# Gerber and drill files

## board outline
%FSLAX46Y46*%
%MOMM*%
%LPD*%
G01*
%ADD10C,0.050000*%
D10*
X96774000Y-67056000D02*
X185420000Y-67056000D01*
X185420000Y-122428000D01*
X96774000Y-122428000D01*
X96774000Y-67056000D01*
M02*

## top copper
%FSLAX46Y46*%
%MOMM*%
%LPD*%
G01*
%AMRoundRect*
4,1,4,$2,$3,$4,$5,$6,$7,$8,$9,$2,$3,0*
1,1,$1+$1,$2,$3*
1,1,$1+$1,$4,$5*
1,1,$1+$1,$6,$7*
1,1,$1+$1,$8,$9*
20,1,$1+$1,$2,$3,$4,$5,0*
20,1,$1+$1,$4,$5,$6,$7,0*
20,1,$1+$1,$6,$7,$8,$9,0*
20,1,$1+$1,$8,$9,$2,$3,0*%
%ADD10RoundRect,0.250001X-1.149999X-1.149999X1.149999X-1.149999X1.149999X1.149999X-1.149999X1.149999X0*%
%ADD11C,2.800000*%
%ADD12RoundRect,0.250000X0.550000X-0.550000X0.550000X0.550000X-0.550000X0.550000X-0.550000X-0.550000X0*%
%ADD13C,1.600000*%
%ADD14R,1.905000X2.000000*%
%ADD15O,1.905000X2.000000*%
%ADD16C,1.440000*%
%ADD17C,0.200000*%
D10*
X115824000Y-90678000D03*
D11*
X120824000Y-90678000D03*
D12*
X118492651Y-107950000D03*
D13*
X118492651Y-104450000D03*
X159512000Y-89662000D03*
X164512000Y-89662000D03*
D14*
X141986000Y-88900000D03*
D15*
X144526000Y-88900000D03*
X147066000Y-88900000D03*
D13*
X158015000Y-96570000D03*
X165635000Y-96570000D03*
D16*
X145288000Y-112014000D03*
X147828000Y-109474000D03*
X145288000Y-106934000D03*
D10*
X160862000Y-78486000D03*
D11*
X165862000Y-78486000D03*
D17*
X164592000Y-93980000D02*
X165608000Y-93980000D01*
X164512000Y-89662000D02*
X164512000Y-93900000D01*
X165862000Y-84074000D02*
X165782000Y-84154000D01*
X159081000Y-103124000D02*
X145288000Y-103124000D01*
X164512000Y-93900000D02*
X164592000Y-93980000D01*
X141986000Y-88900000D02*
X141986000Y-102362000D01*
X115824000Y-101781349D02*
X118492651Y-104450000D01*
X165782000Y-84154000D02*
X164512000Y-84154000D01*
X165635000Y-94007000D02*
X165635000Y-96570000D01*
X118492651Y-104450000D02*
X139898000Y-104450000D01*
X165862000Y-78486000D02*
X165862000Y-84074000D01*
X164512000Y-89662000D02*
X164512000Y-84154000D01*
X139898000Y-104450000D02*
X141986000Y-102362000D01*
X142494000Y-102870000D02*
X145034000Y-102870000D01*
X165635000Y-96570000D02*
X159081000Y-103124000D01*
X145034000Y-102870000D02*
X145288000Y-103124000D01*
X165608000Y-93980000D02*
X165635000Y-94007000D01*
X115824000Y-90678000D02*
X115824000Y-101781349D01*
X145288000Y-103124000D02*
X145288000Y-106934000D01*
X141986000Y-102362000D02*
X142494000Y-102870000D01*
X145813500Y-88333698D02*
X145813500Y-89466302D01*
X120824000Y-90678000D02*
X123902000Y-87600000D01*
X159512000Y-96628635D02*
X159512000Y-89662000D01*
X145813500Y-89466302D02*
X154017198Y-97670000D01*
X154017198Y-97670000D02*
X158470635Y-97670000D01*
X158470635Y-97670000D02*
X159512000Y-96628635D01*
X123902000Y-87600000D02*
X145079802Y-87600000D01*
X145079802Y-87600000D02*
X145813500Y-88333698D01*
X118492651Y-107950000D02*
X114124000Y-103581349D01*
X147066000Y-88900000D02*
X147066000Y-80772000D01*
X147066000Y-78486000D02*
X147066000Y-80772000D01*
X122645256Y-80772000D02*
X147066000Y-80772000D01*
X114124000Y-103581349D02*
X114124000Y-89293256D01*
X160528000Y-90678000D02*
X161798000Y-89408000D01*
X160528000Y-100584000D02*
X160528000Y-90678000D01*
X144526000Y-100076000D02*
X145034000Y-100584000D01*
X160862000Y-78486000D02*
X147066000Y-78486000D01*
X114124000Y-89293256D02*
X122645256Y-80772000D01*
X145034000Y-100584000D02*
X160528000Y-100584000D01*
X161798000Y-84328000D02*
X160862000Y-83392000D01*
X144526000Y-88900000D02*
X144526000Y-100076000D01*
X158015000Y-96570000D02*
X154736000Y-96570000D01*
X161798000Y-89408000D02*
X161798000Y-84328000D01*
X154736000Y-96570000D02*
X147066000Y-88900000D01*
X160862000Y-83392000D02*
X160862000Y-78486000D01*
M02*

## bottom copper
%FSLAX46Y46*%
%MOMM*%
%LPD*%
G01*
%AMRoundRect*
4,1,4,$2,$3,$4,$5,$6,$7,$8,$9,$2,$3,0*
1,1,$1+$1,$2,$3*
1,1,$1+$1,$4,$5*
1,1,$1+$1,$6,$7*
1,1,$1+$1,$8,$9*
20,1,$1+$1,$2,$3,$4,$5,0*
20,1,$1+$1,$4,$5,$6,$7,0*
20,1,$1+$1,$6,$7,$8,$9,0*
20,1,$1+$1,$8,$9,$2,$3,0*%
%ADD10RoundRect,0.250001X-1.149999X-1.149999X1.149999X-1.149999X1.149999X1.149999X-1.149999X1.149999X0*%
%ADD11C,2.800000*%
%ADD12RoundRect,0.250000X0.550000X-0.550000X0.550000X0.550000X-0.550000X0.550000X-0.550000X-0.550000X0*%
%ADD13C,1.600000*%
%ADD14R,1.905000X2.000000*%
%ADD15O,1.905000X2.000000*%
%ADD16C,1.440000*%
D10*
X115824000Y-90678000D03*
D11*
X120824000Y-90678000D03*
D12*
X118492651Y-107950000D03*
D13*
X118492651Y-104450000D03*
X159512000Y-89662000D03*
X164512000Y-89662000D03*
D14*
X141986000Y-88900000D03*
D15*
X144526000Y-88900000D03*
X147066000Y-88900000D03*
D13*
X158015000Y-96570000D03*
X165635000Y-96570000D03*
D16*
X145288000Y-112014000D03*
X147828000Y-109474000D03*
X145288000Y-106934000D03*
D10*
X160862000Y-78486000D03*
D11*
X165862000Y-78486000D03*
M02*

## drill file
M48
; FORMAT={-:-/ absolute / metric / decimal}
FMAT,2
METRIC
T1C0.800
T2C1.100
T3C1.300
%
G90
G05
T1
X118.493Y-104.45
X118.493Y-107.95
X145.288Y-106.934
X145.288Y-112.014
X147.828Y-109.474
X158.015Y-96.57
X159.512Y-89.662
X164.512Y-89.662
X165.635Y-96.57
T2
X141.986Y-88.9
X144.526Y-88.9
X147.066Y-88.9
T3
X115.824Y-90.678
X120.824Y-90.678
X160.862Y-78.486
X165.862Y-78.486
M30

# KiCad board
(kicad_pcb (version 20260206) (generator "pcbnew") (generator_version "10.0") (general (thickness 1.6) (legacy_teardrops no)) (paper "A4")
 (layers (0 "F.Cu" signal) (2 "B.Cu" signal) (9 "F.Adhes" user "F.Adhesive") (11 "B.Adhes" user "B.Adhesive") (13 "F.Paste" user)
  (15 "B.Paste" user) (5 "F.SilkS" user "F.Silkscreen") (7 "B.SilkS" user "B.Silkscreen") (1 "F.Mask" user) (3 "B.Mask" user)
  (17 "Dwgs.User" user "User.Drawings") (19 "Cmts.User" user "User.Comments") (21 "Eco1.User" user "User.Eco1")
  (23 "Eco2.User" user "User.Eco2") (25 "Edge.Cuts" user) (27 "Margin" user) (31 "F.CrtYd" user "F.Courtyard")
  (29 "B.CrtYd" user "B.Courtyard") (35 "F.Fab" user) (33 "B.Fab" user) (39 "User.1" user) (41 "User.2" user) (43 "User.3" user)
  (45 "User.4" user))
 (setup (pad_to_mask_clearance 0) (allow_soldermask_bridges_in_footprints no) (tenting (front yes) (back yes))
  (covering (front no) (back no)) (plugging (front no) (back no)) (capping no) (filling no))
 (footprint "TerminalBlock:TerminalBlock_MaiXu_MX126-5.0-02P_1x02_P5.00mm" (layer "F.Cu") (at 115.824 90.678)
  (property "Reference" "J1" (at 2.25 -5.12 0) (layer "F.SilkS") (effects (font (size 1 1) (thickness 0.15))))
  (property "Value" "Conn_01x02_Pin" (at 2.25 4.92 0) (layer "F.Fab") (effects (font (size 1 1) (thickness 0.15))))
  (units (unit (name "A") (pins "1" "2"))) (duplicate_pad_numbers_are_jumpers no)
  (pad "1" thru_hole roundrect (at 0 0) (size 2.8 2.8) (drill 1.3) (layers "*.Cu" "*.Mask") (remove_unused_layers no)
   (roundrect_rratio 0.089286) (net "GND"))
  (pad "2" thru_hole circle (at 5 0) (size 2.8 2.8) (drill 1.3) (layers "*.Cu" "*.Mask") (remove_unused_layers no) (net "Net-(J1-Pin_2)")))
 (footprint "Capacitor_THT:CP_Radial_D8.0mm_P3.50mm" (layer "F.Cu") (at 118.492651 107.95 90)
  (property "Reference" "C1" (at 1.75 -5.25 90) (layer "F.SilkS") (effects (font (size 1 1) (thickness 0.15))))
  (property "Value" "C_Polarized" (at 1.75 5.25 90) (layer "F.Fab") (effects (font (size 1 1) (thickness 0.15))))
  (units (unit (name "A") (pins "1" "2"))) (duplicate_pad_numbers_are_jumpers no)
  (pad "1" thru_hole roundrect (at 0 0 90) (size 1.6 1.6) (drill 0.8) (layers "*.Cu" "*.Mask") (remove_unused_layers no)
   (roundrect_rratio 0.15625) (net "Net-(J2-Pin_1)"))
  (pad "2" thru_hole circle (at 3.5 0 90) (size 1.6 1.6) (drill 0.8) (layers "*.Cu" "*.Mask") (remove_unused_layers no) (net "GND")))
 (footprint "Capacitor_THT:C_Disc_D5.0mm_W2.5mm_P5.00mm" (layer "F.Cu") (at 159.512 89.662)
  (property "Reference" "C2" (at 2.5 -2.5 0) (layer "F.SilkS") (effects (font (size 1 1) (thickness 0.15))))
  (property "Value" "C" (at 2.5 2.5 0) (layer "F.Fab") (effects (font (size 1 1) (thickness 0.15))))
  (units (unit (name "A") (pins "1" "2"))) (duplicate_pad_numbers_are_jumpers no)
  (pad "1" thru_hole circle (at 0 0) (size 1.6 1.6) (drill 0.8) (layers "*.Cu" "*.Mask") (remove_unused_layers no) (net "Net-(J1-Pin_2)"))
  (pad "2" thru_hole circle (at 5 0) (size 1.6 1.6) (drill 0.8) (layers "*.Cu" "*.Mask") (remove_unused_layers no) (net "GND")))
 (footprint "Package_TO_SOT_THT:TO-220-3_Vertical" (layer "F.Cu") (at 141.986 88.9)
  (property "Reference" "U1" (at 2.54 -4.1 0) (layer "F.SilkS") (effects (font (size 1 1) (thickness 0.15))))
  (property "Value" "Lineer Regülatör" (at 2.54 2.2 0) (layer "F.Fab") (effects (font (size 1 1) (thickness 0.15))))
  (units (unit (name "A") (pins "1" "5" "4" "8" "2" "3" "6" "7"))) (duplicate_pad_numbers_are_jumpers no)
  (pad "1" thru_hole rect (at 0 0) (size 1.905 2) (drill 1.1) (layers "*.Cu" "*.Mask") (remove_unused_layers no) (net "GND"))
  (pad "2" thru_hole oval (at 2.54 0) (size 1.905 2) (drill 1.1) (layers "*.Cu" "*.Mask") (remove_unused_layers no) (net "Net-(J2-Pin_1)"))
  (pad "3" thru_hole oval (at 5.08 0) (size 1.905 2) (drill 1.1) (layers "*.Cu" "*.Mask") (remove_unused_layers no) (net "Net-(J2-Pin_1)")))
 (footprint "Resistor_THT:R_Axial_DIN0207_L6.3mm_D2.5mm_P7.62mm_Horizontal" (layer "F.Cu") (at 158.015 96.57)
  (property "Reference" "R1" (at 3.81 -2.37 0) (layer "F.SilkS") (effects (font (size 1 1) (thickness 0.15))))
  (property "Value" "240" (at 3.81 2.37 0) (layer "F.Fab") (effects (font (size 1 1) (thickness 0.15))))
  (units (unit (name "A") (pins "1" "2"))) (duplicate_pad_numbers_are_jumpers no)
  (pad "1" thru_hole circle (at 0 0) (size 1.6 1.6) (drill 0.8) (layers "*.Cu" "*.Mask") (remove_unused_layers no) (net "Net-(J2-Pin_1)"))
  (pad "2" thru_hole circle (at 7.62 0) (size 1.6 1.6) (drill 0.8) (layers "*.Cu" "*.Mask") (remove_unused_layers no) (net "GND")))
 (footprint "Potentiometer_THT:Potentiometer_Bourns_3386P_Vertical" (layer "F.Cu") (at 145.288 112.014)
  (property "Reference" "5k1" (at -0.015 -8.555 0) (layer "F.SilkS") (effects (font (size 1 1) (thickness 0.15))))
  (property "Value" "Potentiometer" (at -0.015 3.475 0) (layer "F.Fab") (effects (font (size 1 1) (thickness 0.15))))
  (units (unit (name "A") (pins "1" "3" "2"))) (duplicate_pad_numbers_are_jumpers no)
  (pad "1" thru_hole circle (at 0 0) (size 1.44 1.44) (drill 0.8) (layers "*.Cu" "*.Mask") (remove_unused_layers no)
   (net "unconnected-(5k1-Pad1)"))
  (pad "2" thru_hole circle (at 2.54 -2.54) (size 1.44 1.44) (drill 0.8) (layers "*.Cu" "*.Mask") (remove_unused_layers no)
   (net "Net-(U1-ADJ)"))
  (pad "3" thru_hole circle (at 0 -5.08) (size 1.44 1.44) (drill 0.8) (layers "*.Cu" "*.Mask") (remove_unused_layers no) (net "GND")))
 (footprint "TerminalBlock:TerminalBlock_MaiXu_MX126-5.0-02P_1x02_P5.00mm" (layer "F.Cu") (at 160.862 78.486)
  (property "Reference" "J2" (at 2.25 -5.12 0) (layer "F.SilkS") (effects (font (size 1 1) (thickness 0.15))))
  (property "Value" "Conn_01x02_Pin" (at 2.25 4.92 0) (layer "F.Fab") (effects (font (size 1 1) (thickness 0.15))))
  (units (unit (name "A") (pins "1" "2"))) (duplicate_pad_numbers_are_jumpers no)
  (pad "1" thru_hole roundrect (at 0 0) (size 2.8 2.8) (drill 1.3) (layers "*.Cu" "*.Mask") (remove_unused_layers no)
   (roundrect_rratio 0.089286) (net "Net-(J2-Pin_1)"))
  (pad "2" thru_hole circle (at 5 0) (size 2.8 2.8) (drill 1.3) (layers "*.Cu" "*.Mask") (remove_unused_layers no) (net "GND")))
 (gr_rect (start 96.774 67.056) (end 185.42 122.428) (stroke (width 0.05) (type default)) (fill no) (layer "Edge.Cuts"))
 (segment (start 164.592 93.98) (end 165.608 93.98) (width 0.2) (layer "F.Cu") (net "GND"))
 (segment (start 164.512 89.662) (end 164.512 93.9) (width 0.2) (layer "F.Cu") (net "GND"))
 (segment (start 165.862 84.074) (end 165.782 84.154) (width 0.2) (layer "F.Cu") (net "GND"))
 (segment (start 159.081 103.124) (end 145.288 103.124) (width 0.2) (layer "F.Cu") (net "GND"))
 (segment (start 164.512 93.9) (end 164.592 93.98) (width 0.2) (layer "F.Cu") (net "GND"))
 (segment (start 141.986 88.9) (end 141.986 102.362) (width 0.2) (layer "F.Cu") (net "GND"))
 (segment (start 115.824 101.781349) (end 118.492651 104.45) (width 0.2) (layer "F.Cu") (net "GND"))
 (segment (start 165.782 84.154) (end 164.512 84.154) (width 0.2) (layer "F.Cu") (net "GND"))
 (segment (start 165.635 94.007) (end 165.635 96.57) (width 0.2) (layer "F.Cu") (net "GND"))
 (segment (start 118.492651 104.45) (end 139.898 104.45) (width 0.2) (layer "F.Cu") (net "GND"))
 (segment (start 165.862 78.486) (end 165.862 84.074) (width 0.2) (layer "F.Cu") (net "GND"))
 (segment (start 164.512 89.662) (end 164.512 84.154) (width 0.2) (layer "F.Cu") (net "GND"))
 (segment (start 139.898 104.45) (end 141.986 102.362) (width 0.2) (layer "F.Cu") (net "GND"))
 (segment (start 142.494 102.87) (end 145.034 102.87) (width 0.2) (layer "F.Cu") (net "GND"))
 (segment (start 165.635 96.57) (end 159.081 103.124) (width 0.2) (layer "F.Cu") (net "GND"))
 (segment (start 145.034 102.87) (end 145.288 103.124) (width 0.2) (layer "F.Cu") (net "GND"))
 (segment (start 165.608 93.98) (end 165.635 94.007) (width 0.2) (layer "F.Cu") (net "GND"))
 (segment (start 115.824 90.678) (end 115.824 101.781349) (width 0.2) (layer "F.Cu") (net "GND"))
 (segment (start 145.288 103.124) (end 145.288 106.934) (width 0.2) (layer "F.Cu") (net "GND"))
 (segment (start 141.986 102.362) (end 142.494 102.87) (width 0.2) (layer "F.Cu") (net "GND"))
 (segment (start 145.8135 88.333698) (end 145.8135 89.466302) (width 0.2) (layer "F.Cu") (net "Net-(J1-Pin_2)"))
 (segment (start 120.824 90.678) (end 123.902 87.6) (width 0.2) (layer "F.Cu") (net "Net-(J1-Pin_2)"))
 (segment (start 159.512 96.628635) (end 159.512 89.662) (width 0.2) (layer "F.Cu") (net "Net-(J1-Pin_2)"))
 (segment (start 145.8135 89.466302) (end 154.017198 97.67) (width 0.2) (layer "F.Cu") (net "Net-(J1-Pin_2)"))
 (segment (start 154.017198 97.67) (end 158.470635 97.67) (width 0.2) (layer "F.Cu") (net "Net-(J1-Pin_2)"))
 (segment (start 158.470635 97.67) (end 159.512 96.628635) (width 0.2) (layer "F.Cu") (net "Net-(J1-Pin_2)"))
 (segment (start 123.902 87.6) (end 145.079802 87.6) (width 0.2) (layer "F.Cu") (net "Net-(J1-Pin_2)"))
 (segment (start 145.079802 87.6) (end 145.8135 88.333698) (width 0.2) (layer "F.Cu") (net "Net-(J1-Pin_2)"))
 (segment (start 118.492651 107.95) (end 114.124 103.581349) (width 0.2) (layer "F.Cu") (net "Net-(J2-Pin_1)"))
 (segment (start 147.066 88.9) (end 147.066 80.772) (width 0.2) (layer "F.Cu") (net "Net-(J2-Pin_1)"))
 (segment (start 147.066 78.486) (end 147.066 80.772) (width 0.2) (layer "F.Cu") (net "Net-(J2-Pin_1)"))
 (segment (start 122.645256 80.772) (end 147.066 80.772) (width 0.2) (layer "F.Cu") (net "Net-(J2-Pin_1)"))
 (segment (start 114.124 103.581349) (end 114.124 89.293256) (width 0.2) (layer "F.Cu") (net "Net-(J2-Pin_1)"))
 (segment (start 160.528 90.678) (end 161.798 89.408) (width 0.2) (layer "F.Cu") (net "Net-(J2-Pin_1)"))
 (segment (start 160.528 100.584) (end 160.528 90.678) (width 0.2) (layer "F.Cu") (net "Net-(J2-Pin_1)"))
 (segment (start 144.526 100.076) (end 145.034 100.584) (width 0.2) (layer "F.Cu") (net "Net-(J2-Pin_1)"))
 (segment (start 160.862 78.486) (end 147.066 78.486) (width 0.2) (layer "F.Cu") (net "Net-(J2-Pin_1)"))
 (segment (start 114.124 89.293256) (end 122.645256 80.772) (width 0.2) (layer "F.Cu") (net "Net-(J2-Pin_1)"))
 (segment (start 145.034 100.584) (end 160.528 100.584) (width 0.2) (layer "F.Cu") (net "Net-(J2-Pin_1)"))
 (segment (start 161.798 84.328) (end 160.862 83.392) (width 0.2) (layer "F.Cu") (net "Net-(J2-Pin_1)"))
 (segment (start 144.526 88.9) (end 144.526 100.076) (width 0.2) (layer "F.Cu") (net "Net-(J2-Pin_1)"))
 (segment (start 158.015 96.57) (end 154.736 96.57) (width 0.2) (layer "F.Cu") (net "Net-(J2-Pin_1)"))
 (segment (start 161.798 89.408) (end 161.798 84.328) (width 0.2) (layer "F.Cu") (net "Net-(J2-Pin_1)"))
 (segment (start 154.736 96.57) (end 147.066 88.9) (width 0.2) (layer "F.Cu") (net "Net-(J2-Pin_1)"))
 (segment (start 160.862 83.392) (end 160.862 78.486) (width 0.2) (layer "F.Cu") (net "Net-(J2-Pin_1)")))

